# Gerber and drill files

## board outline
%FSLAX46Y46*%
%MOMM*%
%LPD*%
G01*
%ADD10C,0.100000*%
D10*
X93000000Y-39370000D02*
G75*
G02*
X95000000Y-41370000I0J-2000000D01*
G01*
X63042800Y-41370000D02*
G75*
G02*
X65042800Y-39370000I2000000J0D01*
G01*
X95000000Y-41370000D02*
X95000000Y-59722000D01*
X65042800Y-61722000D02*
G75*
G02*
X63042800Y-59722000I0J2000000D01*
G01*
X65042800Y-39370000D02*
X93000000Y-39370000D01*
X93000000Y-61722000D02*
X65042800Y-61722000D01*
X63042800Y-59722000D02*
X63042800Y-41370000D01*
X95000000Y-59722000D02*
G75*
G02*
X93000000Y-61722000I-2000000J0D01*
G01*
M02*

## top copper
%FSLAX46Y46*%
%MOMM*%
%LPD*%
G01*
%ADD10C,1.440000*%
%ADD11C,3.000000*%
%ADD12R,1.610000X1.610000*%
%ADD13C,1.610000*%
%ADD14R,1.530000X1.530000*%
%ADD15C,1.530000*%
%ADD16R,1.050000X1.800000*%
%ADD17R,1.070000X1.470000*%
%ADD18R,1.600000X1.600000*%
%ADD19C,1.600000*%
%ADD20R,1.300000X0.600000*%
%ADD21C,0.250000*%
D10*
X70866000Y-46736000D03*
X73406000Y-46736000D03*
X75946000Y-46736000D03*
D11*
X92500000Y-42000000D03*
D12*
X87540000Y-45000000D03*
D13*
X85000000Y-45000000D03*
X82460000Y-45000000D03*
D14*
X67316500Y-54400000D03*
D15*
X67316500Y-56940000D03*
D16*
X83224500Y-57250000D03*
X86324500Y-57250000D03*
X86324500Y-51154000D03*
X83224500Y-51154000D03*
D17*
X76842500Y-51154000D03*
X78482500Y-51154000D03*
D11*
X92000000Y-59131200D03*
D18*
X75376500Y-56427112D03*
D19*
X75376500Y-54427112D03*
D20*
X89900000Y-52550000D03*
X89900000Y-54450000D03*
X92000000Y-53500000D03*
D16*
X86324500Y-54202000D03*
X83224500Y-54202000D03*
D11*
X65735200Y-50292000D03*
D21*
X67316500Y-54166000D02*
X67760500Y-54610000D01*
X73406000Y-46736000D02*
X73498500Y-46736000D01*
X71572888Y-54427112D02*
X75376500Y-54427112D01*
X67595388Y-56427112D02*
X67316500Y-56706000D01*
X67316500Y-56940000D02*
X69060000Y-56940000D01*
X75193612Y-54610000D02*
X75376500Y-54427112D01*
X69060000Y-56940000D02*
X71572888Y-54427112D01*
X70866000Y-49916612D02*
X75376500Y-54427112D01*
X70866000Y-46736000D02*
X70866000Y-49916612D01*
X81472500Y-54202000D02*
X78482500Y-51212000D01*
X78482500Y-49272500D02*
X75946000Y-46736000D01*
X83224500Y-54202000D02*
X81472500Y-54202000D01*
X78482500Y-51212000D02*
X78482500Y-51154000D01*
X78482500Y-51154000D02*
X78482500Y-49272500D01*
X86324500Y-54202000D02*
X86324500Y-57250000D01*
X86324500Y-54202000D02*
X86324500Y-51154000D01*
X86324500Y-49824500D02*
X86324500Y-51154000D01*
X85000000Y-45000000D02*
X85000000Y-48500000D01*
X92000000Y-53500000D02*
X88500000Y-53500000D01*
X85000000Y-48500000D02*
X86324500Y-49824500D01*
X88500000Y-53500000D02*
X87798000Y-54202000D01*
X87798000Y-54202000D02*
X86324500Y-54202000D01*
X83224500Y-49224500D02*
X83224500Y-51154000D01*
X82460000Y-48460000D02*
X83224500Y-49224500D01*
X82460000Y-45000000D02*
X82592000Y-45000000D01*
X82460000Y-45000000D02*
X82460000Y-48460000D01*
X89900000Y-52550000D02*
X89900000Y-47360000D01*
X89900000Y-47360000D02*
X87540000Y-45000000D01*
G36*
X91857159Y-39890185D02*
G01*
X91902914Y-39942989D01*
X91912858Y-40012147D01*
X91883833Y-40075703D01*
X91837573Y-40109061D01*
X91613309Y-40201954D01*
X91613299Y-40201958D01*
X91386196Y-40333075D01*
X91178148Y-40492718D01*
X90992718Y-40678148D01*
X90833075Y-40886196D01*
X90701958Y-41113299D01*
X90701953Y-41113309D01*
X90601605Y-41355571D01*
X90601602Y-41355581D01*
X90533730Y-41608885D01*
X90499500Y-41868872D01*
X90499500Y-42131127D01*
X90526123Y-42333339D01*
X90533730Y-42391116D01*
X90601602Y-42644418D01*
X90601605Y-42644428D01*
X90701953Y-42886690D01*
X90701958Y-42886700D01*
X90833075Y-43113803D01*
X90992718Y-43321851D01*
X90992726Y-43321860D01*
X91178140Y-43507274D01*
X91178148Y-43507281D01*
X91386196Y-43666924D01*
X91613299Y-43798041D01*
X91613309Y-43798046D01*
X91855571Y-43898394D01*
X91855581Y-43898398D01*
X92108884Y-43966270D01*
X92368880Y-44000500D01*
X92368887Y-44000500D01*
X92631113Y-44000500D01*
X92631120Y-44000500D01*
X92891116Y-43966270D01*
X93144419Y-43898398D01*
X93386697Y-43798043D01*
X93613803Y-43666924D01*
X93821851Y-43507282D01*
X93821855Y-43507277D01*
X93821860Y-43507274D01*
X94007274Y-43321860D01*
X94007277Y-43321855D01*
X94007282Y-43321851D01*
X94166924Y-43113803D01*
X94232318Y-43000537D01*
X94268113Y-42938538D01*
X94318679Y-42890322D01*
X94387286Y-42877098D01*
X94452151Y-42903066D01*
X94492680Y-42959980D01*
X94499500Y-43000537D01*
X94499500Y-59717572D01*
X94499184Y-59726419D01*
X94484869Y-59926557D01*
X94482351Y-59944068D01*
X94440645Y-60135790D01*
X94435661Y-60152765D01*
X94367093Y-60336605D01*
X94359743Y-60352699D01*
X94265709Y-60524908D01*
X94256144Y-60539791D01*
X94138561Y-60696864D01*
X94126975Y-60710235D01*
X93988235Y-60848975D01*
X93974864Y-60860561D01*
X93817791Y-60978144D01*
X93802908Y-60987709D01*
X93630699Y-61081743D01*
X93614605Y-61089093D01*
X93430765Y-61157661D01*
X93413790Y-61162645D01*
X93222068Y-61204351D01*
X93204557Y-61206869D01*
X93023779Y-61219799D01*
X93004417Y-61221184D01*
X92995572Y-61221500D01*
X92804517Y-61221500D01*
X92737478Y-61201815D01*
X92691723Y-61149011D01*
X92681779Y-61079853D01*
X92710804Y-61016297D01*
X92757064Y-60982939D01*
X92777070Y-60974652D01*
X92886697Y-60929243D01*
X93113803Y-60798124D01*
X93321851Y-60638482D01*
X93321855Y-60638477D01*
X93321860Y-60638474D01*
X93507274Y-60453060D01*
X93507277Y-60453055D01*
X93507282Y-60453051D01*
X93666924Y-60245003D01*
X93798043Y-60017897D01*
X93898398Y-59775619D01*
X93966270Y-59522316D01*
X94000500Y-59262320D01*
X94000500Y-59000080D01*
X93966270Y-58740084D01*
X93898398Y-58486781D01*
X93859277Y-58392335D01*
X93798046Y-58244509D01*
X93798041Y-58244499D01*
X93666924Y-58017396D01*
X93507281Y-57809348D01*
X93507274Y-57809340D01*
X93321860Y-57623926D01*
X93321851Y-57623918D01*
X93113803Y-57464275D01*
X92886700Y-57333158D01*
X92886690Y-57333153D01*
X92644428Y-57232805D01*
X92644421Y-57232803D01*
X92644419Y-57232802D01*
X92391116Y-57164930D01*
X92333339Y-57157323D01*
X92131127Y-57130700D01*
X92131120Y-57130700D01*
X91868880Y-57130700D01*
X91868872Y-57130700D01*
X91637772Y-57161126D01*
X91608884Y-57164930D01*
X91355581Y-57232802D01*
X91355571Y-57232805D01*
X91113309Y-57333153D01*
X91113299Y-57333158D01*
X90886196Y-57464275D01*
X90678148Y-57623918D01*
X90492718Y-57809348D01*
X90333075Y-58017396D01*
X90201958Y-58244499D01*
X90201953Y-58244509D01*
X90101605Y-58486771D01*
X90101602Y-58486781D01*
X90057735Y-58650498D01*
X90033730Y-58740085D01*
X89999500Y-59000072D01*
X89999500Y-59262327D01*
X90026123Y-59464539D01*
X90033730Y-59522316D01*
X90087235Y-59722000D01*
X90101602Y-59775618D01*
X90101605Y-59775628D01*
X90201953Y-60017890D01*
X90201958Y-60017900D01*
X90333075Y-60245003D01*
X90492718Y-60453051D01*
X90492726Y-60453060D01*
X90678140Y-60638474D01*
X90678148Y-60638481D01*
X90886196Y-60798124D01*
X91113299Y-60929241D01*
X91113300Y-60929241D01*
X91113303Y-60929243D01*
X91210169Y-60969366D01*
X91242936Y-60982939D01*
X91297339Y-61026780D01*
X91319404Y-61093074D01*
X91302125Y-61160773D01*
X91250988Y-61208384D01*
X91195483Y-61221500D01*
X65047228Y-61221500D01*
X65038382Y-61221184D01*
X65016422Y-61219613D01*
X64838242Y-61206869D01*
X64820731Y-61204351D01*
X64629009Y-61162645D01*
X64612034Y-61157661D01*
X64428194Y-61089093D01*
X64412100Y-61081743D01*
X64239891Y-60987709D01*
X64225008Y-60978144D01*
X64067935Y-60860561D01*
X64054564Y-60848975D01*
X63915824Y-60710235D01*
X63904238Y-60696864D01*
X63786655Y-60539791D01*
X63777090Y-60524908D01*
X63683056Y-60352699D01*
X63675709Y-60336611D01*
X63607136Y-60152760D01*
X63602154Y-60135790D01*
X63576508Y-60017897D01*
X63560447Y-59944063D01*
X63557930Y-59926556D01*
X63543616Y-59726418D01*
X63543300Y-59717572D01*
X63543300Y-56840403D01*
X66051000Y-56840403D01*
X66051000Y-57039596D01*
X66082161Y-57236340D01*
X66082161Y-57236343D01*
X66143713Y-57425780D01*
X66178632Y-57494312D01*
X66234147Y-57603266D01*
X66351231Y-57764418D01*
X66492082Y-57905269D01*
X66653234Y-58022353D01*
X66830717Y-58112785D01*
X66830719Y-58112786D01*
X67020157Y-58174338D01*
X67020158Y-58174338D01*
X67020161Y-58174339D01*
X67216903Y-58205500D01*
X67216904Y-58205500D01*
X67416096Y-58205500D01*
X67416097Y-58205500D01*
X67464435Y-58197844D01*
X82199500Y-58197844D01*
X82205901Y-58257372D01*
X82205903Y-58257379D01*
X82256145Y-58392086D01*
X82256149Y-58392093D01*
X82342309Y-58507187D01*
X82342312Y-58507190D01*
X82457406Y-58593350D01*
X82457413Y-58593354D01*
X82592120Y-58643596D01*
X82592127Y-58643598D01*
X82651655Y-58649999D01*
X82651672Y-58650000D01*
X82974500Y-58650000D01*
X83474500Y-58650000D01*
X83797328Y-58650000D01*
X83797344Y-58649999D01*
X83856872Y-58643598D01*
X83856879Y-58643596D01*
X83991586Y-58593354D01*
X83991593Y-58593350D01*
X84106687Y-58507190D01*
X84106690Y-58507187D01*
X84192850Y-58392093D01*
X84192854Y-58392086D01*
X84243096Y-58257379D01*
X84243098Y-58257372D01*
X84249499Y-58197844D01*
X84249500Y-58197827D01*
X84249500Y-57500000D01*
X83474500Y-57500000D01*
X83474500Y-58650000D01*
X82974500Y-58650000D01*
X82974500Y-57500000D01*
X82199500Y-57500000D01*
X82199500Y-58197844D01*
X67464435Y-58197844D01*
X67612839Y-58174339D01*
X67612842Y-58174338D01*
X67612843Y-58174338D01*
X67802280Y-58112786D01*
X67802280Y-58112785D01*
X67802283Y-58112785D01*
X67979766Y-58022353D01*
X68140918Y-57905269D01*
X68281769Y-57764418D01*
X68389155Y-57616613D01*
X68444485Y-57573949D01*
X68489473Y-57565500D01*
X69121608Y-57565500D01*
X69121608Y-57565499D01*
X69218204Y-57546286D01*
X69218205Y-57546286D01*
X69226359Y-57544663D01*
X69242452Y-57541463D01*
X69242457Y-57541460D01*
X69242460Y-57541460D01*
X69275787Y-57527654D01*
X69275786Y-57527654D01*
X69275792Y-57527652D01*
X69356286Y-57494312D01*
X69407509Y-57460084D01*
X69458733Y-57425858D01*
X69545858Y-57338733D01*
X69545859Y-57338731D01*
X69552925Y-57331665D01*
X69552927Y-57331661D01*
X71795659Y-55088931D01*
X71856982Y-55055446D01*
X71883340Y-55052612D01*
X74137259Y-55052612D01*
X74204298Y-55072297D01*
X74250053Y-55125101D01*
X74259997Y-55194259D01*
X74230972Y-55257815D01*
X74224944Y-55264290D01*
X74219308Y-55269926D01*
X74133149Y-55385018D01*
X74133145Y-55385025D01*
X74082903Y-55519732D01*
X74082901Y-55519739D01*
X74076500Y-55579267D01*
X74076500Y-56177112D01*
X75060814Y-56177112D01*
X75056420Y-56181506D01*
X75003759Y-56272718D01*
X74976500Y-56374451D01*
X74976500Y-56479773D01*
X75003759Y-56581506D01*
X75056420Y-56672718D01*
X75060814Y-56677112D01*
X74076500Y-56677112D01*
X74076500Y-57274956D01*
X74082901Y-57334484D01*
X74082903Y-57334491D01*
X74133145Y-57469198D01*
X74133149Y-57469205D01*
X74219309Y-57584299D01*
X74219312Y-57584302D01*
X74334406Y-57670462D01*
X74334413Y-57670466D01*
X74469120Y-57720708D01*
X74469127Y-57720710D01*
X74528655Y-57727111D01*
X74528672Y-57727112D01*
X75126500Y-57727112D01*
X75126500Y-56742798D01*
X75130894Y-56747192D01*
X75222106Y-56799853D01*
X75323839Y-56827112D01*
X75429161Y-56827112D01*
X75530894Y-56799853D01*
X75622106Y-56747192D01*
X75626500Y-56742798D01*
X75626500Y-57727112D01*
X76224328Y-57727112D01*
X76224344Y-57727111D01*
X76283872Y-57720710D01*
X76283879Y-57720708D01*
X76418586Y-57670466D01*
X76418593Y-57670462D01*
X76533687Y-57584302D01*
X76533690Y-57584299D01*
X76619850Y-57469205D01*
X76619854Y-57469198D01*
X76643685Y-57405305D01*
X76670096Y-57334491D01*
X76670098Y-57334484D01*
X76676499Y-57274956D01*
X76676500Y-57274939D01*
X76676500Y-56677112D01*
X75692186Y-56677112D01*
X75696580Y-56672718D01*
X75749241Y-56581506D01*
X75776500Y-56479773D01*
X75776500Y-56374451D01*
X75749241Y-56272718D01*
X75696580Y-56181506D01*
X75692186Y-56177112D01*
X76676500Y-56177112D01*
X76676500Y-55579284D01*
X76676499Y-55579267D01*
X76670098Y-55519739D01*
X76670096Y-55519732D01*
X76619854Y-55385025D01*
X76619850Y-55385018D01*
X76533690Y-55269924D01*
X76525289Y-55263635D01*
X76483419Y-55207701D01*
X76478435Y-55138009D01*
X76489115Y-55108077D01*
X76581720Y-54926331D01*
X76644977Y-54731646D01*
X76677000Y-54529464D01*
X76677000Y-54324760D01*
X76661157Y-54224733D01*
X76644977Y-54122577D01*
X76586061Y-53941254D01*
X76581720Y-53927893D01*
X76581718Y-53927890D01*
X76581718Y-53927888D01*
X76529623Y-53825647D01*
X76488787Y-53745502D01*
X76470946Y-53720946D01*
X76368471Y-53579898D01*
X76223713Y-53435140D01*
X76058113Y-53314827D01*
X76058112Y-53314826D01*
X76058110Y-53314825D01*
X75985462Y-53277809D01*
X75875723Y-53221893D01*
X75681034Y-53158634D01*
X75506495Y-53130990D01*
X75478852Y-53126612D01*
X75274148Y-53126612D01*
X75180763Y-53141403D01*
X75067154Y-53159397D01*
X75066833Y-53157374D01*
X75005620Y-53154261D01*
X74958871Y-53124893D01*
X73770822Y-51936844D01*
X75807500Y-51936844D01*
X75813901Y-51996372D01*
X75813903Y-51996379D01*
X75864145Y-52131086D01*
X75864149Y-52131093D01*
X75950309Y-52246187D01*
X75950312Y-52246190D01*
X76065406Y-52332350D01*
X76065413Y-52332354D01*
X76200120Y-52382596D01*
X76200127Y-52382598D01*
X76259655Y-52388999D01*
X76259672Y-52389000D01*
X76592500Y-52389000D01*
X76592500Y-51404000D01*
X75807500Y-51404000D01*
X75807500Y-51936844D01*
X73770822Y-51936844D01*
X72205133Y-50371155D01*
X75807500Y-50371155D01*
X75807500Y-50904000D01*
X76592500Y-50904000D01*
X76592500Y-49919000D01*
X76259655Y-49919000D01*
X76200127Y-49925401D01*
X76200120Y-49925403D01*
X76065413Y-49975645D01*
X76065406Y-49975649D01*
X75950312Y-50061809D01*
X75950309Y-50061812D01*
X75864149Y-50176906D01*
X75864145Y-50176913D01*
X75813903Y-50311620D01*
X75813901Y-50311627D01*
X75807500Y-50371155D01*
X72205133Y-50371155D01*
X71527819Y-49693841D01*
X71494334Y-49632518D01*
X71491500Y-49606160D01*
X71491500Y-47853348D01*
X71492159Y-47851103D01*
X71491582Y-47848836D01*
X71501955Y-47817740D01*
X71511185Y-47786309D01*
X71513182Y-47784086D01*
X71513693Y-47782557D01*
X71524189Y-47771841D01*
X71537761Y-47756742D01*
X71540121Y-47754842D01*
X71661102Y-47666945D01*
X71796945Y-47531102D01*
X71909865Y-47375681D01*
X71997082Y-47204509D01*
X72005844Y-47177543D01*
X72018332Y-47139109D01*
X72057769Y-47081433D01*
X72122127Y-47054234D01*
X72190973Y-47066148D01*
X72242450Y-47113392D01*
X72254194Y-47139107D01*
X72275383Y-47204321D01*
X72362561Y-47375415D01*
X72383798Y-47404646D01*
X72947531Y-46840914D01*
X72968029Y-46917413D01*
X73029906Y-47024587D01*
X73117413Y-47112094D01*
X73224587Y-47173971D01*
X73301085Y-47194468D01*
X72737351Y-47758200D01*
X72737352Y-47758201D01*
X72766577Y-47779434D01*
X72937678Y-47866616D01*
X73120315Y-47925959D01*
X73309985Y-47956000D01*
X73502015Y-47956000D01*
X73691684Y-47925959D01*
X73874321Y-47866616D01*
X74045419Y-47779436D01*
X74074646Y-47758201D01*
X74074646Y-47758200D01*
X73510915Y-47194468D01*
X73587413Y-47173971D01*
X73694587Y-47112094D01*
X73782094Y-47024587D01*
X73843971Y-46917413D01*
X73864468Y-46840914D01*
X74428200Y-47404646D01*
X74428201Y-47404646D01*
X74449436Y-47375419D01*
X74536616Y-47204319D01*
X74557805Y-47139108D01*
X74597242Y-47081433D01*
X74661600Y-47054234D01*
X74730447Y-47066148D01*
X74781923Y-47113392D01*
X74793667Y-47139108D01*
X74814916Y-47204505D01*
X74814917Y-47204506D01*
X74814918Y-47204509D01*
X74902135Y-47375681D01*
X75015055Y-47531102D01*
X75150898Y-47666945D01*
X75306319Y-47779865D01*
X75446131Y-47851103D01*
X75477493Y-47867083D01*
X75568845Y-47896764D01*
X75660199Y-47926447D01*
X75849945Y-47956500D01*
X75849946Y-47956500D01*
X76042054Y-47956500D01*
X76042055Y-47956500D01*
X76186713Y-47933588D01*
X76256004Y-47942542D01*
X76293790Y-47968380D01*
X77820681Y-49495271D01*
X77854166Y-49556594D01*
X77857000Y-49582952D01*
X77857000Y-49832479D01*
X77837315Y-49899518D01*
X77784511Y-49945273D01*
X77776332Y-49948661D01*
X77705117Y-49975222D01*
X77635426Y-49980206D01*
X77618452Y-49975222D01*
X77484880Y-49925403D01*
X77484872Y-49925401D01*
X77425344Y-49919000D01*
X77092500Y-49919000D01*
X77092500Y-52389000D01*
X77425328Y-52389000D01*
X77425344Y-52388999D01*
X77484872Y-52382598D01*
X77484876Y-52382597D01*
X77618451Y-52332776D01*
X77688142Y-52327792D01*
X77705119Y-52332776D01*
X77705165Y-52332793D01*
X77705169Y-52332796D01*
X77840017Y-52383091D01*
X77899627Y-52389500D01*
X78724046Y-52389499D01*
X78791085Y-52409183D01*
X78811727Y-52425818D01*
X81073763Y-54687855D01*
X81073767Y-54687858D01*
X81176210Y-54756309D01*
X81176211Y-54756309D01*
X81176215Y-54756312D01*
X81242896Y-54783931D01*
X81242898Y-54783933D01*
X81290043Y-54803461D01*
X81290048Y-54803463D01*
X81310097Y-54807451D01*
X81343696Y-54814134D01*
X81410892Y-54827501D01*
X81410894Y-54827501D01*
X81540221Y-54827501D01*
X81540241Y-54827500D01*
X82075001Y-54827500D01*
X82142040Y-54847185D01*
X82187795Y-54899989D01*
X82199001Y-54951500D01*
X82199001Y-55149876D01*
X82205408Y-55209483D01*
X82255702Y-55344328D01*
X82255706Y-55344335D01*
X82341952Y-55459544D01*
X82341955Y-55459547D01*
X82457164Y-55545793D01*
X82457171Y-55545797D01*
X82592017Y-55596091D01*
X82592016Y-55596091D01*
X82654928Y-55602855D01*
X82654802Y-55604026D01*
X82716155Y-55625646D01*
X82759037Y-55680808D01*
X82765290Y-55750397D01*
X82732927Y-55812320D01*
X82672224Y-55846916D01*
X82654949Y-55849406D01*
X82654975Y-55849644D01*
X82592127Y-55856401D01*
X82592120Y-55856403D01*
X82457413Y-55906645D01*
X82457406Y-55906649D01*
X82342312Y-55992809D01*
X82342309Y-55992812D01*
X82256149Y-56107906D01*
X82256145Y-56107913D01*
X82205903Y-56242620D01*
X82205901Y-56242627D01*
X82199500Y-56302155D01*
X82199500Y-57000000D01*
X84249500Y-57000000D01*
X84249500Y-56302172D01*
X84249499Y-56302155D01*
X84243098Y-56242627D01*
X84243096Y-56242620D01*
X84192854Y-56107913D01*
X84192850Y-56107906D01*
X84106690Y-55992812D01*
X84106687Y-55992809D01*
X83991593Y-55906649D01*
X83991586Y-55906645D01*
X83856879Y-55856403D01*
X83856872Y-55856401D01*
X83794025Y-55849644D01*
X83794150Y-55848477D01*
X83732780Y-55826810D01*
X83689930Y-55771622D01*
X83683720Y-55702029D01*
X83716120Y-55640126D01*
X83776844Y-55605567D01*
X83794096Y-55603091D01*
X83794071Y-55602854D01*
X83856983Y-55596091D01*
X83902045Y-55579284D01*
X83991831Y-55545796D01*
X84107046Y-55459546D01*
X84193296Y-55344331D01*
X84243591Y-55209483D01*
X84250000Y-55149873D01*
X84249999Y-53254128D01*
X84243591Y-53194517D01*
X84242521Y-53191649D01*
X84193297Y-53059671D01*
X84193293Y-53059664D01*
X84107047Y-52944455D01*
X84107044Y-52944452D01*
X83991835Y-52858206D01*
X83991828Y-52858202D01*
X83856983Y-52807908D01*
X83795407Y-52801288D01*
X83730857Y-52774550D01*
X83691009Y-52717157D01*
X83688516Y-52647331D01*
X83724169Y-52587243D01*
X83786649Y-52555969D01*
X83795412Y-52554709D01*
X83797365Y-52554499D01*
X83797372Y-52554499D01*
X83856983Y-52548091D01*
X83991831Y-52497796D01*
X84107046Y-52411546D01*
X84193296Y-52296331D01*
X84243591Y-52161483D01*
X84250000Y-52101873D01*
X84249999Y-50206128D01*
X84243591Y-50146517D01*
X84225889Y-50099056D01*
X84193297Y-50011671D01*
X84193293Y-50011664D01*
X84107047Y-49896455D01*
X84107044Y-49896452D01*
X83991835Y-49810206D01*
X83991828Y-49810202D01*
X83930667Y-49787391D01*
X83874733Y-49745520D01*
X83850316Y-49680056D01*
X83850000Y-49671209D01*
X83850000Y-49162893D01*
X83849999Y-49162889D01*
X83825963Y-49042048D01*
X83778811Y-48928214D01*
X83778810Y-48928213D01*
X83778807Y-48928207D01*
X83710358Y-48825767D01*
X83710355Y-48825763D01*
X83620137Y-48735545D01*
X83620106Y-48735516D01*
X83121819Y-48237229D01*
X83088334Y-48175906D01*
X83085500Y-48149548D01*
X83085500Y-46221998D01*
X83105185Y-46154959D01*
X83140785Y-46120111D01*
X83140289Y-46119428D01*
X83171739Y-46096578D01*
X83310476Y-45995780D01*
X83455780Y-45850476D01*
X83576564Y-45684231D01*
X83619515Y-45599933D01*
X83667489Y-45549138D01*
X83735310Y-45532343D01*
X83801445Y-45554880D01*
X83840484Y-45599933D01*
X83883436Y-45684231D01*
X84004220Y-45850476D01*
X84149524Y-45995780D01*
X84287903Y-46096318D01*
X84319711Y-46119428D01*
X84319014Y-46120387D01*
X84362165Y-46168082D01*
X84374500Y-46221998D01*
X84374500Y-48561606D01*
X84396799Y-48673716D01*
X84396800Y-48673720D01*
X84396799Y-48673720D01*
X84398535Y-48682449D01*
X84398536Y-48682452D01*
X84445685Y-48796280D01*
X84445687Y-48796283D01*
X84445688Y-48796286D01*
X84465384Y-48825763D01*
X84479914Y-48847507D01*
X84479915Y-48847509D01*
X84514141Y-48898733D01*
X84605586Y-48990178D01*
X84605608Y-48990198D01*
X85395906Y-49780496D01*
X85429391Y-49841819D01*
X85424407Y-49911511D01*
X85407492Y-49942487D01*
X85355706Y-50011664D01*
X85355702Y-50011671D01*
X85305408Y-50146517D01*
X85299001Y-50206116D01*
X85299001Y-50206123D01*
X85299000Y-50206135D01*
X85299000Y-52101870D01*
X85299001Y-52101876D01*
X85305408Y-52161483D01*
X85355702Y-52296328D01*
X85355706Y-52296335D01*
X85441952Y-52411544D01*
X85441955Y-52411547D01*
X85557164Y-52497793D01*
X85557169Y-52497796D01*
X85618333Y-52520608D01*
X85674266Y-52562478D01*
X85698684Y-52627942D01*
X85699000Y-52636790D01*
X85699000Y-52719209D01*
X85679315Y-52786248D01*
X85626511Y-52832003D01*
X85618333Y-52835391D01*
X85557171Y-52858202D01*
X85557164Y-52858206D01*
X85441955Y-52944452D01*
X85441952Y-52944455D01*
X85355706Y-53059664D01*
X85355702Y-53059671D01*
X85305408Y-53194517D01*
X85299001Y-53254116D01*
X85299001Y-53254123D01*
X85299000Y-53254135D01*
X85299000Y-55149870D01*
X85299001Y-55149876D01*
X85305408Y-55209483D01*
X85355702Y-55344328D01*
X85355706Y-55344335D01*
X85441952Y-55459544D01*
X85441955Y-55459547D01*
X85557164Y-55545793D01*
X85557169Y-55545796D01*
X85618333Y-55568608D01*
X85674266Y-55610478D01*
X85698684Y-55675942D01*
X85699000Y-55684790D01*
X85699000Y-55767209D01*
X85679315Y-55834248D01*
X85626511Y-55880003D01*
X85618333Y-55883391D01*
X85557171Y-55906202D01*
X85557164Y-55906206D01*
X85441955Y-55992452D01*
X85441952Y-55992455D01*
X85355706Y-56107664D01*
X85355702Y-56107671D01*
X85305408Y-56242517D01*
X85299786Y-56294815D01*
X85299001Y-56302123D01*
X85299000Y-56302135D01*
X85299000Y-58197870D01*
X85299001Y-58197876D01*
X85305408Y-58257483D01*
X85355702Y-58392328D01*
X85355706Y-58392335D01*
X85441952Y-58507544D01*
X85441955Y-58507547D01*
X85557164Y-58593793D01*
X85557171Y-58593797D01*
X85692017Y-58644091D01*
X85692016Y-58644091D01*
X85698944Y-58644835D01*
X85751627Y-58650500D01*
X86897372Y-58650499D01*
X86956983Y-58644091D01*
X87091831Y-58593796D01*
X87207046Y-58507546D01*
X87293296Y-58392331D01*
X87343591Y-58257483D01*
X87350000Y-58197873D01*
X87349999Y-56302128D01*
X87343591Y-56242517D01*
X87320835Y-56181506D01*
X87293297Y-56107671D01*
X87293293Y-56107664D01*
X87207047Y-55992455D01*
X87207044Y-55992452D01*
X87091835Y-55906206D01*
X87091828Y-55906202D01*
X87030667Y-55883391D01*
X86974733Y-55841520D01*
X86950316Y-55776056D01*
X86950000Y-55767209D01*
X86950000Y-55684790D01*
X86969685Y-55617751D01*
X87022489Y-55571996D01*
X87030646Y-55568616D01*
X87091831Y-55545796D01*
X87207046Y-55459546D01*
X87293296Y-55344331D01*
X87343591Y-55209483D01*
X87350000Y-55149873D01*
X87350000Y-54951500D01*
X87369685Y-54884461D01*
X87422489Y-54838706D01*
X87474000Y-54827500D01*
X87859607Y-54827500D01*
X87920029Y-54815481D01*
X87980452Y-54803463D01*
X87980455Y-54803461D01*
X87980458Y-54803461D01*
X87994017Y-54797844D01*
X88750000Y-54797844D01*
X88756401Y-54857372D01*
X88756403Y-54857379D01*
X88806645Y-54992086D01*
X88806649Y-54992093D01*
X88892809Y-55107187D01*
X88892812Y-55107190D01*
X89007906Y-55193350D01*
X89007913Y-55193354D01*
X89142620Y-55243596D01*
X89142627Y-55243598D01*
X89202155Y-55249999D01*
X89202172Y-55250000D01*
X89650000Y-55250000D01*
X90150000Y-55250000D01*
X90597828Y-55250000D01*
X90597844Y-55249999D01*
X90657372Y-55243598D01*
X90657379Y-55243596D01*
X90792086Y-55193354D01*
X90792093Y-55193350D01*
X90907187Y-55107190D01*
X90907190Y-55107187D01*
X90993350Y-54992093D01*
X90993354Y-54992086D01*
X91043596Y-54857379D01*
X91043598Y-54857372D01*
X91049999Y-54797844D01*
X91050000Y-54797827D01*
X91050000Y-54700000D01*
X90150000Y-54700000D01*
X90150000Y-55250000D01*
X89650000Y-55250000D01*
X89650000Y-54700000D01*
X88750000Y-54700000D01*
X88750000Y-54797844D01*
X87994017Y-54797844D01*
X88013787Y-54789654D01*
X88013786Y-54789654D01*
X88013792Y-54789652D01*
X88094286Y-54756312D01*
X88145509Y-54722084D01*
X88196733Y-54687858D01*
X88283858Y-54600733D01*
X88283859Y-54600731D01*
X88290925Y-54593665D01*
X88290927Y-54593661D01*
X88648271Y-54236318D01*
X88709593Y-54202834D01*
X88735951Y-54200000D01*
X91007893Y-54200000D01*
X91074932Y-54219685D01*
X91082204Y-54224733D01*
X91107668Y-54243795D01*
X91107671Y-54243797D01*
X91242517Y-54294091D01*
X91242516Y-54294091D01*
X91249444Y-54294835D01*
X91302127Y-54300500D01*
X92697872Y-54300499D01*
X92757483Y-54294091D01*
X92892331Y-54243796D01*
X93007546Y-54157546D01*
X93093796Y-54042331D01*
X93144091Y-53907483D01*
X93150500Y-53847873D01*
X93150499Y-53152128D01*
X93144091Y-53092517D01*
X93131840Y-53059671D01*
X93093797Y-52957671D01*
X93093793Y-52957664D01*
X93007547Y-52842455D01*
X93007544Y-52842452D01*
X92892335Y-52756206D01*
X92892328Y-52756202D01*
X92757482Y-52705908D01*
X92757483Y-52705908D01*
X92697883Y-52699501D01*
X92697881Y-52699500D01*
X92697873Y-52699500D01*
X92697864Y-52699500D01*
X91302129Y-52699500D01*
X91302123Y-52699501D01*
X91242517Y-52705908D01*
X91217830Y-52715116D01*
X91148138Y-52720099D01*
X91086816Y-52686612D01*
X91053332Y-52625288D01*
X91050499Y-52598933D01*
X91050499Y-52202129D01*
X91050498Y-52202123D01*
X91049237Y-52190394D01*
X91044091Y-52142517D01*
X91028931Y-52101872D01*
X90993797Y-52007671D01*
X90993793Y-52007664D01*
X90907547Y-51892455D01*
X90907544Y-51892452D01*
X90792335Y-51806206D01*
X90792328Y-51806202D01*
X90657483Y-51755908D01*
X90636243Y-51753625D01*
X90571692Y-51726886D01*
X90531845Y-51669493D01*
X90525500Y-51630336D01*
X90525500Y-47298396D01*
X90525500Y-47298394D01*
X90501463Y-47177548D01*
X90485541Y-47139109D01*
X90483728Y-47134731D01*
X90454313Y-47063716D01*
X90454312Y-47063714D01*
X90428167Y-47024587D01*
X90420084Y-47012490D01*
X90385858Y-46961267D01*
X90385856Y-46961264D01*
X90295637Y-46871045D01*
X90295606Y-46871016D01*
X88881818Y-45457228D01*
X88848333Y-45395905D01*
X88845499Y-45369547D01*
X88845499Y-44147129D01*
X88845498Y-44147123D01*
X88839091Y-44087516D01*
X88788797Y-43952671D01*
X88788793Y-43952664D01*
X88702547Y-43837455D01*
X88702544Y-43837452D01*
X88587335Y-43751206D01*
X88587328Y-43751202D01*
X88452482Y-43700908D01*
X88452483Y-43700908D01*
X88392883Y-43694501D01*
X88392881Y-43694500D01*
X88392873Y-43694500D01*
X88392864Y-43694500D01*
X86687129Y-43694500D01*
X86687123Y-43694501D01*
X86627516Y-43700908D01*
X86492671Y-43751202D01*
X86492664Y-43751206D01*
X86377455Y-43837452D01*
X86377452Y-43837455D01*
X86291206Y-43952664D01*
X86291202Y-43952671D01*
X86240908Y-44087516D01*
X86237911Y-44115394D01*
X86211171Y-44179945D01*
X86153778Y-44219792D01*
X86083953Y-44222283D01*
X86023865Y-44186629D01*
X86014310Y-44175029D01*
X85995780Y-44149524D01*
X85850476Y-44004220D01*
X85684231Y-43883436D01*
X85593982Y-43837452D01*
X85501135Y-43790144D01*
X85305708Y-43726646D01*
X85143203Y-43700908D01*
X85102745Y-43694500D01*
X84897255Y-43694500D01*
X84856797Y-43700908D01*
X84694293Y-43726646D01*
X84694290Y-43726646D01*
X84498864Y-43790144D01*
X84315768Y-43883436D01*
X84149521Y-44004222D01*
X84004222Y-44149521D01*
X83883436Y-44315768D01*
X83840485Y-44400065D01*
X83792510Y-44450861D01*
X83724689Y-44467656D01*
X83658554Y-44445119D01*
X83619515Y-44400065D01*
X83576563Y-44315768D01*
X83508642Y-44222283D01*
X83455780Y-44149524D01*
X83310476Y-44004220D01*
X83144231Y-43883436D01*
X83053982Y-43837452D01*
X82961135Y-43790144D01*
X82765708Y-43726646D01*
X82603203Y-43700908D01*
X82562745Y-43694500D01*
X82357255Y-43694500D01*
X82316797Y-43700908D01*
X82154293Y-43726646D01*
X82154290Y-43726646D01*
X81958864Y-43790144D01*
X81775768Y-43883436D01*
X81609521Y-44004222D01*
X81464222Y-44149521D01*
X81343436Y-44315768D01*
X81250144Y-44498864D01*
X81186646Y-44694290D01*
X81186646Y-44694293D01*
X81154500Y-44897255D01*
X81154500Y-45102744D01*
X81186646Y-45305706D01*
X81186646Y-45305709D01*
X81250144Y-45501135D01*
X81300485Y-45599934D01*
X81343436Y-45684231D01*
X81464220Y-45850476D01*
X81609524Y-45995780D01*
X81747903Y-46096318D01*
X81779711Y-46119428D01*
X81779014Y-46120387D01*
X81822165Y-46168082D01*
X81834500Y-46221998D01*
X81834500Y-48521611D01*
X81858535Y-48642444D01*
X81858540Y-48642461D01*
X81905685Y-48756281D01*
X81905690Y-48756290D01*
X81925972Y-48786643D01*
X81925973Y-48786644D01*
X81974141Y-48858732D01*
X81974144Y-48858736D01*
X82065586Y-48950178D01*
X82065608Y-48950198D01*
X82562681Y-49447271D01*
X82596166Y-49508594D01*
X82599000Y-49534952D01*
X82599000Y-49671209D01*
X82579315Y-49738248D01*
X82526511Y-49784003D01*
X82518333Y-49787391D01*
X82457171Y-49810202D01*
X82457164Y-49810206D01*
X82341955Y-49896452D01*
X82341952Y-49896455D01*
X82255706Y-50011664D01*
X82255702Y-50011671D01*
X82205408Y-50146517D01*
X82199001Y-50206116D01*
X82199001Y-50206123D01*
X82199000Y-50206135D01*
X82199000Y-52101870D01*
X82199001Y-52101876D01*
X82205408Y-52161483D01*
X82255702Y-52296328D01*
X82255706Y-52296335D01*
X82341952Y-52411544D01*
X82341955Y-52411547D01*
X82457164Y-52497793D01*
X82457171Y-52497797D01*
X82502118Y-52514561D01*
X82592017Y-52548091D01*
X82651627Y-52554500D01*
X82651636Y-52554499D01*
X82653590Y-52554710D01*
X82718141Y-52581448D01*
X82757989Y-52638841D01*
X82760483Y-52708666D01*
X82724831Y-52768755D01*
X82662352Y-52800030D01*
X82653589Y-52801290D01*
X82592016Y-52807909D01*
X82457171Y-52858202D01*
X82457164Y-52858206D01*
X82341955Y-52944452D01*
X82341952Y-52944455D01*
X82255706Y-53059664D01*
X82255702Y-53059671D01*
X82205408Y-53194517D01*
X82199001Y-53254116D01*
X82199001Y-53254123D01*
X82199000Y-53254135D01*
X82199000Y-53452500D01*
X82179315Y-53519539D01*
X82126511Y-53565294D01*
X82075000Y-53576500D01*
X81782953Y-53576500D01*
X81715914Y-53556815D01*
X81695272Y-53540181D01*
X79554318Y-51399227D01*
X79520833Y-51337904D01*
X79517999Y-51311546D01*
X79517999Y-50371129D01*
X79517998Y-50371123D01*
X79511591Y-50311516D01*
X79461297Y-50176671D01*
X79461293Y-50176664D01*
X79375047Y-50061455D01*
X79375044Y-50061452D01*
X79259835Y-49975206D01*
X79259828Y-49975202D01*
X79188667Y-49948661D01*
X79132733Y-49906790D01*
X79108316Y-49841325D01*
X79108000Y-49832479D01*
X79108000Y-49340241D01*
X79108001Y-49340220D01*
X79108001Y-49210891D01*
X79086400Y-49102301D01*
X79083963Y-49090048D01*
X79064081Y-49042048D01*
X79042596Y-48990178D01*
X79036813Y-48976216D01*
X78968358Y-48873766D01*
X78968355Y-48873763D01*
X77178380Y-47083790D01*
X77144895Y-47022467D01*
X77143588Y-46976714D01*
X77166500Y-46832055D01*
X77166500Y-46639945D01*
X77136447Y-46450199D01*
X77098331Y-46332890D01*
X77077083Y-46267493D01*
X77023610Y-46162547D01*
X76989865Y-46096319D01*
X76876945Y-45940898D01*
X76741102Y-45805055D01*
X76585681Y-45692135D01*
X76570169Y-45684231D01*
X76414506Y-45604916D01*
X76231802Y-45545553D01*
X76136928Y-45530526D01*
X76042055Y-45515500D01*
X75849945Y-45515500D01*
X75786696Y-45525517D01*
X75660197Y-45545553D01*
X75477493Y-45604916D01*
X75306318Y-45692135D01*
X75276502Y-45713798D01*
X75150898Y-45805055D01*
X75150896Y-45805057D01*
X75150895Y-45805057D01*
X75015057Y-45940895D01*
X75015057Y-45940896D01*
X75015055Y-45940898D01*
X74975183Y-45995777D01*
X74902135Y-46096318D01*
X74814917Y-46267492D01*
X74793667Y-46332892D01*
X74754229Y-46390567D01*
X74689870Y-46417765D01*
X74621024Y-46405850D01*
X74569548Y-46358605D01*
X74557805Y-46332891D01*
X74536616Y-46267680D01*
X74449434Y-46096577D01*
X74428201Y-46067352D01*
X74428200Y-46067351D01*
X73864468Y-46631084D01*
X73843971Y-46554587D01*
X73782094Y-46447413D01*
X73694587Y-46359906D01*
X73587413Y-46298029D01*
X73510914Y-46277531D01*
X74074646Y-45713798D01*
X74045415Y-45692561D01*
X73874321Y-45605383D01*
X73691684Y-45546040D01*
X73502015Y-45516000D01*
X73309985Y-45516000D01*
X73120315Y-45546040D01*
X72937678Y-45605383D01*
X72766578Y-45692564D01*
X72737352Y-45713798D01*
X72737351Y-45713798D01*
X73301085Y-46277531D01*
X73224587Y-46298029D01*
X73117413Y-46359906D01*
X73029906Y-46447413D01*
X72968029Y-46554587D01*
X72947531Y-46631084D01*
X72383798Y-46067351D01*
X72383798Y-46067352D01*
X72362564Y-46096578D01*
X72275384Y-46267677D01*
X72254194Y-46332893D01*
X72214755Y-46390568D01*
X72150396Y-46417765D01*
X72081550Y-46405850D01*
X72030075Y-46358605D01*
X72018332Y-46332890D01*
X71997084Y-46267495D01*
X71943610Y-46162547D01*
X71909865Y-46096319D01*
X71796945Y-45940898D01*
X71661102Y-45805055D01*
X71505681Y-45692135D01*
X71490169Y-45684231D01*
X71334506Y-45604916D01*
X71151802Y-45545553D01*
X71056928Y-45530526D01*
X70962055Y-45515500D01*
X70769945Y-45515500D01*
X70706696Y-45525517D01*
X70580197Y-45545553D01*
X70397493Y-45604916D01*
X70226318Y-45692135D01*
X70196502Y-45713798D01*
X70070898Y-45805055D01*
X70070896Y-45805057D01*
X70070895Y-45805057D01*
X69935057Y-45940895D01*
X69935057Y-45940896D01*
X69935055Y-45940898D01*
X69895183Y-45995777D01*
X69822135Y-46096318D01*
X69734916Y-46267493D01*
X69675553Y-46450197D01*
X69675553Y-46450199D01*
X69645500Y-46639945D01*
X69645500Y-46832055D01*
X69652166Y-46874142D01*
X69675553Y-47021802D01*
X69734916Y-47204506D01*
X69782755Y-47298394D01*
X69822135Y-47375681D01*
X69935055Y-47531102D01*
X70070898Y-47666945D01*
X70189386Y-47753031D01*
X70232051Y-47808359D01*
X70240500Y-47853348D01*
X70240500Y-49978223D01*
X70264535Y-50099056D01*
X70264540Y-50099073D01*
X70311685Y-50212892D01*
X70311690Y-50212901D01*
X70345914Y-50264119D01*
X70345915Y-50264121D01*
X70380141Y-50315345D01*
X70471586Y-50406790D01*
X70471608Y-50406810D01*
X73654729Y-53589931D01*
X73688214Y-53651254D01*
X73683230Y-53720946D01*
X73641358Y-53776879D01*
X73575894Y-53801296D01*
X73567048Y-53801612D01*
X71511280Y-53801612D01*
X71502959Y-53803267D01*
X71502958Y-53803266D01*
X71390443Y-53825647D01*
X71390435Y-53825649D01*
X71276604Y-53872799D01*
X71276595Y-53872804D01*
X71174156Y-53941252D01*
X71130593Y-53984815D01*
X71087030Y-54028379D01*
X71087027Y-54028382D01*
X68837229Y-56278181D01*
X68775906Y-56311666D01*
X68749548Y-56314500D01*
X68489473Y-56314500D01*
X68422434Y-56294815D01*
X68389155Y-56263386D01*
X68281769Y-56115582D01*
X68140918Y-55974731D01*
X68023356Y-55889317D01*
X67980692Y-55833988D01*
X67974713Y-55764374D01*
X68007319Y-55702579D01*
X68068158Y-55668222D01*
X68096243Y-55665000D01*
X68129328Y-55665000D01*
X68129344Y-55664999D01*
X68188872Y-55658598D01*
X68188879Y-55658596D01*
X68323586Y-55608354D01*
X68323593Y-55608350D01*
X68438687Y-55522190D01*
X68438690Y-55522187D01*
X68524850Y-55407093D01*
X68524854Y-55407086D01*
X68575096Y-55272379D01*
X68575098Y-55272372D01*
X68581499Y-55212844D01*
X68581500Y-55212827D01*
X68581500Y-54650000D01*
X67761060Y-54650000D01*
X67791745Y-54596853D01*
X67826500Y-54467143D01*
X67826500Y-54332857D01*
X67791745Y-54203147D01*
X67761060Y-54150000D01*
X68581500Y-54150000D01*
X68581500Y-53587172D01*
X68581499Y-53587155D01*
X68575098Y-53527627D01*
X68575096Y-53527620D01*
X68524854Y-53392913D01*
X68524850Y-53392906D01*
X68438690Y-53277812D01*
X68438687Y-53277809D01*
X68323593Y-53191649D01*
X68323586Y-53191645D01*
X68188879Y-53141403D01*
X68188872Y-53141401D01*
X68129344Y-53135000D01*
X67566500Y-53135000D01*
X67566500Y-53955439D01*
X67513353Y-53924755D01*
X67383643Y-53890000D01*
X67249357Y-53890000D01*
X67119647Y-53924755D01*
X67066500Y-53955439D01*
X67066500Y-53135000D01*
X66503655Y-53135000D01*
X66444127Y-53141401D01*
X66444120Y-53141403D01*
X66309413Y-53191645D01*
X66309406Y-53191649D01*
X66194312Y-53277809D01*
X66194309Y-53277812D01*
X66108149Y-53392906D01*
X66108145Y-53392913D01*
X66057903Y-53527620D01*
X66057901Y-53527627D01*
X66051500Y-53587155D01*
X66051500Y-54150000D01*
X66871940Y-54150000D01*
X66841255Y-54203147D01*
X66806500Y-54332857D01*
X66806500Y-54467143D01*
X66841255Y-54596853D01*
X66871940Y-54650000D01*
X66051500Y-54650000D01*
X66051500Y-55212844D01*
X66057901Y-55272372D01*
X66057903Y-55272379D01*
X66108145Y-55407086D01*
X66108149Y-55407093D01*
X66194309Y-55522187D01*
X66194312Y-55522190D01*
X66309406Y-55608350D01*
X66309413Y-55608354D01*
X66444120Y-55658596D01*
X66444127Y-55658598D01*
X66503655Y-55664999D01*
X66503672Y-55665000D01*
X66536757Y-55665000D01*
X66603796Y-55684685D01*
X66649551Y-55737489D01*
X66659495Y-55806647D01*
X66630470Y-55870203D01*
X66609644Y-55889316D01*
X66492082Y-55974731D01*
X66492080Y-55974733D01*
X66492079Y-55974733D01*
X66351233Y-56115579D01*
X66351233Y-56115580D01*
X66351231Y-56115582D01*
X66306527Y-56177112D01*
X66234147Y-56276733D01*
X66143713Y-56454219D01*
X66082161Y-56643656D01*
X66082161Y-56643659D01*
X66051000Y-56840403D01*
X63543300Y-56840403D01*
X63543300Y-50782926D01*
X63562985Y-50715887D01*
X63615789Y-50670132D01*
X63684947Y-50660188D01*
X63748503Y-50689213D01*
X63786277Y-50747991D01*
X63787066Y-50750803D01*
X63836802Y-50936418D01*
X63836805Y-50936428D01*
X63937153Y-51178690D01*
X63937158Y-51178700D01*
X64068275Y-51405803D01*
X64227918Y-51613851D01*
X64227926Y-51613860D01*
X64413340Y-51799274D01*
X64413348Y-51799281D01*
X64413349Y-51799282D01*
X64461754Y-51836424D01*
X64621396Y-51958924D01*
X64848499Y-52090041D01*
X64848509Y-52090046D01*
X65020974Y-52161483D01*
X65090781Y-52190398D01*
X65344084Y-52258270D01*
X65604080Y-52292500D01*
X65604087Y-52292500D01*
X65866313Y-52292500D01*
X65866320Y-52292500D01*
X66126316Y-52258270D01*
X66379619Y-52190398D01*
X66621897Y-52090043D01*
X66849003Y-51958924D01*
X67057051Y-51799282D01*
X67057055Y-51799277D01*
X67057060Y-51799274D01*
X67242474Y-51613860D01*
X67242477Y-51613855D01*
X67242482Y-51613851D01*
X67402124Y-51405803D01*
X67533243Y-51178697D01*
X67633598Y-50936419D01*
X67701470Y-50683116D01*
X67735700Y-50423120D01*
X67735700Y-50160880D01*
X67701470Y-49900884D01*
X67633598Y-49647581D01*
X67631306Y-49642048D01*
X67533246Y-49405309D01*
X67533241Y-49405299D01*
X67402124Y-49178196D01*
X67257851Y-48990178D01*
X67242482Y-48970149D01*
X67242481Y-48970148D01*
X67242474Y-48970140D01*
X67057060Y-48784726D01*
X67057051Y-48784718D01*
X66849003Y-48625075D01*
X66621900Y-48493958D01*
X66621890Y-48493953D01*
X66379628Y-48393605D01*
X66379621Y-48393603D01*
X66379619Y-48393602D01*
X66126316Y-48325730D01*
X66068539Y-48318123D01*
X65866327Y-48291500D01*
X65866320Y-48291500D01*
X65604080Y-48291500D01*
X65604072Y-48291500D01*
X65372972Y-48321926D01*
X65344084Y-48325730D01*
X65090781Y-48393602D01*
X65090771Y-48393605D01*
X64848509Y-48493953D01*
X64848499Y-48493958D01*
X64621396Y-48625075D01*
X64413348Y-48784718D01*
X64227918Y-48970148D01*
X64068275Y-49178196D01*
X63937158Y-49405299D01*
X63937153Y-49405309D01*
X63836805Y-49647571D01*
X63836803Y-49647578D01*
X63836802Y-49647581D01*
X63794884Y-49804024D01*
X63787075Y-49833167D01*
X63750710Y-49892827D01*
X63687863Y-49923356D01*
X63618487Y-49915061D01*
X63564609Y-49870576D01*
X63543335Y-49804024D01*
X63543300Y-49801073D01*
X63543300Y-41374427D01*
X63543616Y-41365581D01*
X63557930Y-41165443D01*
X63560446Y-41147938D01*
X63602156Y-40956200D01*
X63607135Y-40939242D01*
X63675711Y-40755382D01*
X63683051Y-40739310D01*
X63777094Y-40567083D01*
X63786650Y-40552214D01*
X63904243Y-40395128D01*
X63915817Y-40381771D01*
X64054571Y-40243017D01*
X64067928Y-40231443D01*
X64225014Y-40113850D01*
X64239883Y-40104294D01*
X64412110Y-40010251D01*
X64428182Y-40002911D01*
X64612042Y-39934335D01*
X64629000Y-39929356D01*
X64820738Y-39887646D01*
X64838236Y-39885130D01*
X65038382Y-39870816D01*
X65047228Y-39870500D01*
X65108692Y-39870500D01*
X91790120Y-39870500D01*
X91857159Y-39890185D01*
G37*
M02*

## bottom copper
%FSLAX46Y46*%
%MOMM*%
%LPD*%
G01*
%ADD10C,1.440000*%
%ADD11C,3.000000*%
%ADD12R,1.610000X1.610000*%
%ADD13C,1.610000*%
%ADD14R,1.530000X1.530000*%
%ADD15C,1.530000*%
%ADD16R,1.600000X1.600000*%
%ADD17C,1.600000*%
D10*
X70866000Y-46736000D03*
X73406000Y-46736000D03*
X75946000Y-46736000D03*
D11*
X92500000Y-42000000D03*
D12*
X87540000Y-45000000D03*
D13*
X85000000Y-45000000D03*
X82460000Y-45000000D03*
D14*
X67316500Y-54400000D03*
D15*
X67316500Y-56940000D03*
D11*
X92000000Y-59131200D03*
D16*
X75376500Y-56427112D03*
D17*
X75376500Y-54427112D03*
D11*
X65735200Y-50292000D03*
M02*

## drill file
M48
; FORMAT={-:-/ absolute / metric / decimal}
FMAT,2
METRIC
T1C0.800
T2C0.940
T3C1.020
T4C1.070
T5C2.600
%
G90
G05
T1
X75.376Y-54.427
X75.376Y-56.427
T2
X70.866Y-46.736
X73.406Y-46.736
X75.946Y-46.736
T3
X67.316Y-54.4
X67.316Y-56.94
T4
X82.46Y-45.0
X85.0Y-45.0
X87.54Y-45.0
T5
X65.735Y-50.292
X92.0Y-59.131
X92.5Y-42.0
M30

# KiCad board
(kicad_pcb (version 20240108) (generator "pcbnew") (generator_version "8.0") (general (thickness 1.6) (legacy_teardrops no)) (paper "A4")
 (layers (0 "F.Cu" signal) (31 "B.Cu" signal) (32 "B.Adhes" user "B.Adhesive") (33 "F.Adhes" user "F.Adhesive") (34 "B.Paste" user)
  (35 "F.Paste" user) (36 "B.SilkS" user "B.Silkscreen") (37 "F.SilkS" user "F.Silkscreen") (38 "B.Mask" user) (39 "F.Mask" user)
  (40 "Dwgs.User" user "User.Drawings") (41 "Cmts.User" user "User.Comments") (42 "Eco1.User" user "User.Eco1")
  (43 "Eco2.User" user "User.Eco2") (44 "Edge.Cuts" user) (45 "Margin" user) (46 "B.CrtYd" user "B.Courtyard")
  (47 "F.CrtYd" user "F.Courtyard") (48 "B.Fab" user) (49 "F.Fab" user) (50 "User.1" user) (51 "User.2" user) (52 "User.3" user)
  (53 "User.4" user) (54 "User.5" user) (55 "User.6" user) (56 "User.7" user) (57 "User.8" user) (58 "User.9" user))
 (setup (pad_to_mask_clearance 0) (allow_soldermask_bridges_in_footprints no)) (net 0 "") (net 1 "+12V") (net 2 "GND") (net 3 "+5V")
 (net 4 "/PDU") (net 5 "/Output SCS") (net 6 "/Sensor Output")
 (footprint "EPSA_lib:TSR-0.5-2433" (layer "F.Cu") (at 67.656 48.736)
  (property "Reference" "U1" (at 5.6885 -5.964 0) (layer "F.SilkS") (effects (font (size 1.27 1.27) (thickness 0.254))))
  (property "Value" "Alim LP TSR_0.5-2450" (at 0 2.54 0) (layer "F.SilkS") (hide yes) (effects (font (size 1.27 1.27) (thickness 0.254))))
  (pad "1" thru_hole circle (at 3.21 -2) (size 1.44 1.44) (drill 0.94) (layers "*.Cu" "*.Mask") (remove_unused_layers no) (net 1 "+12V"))
  (pad "2" thru_hole circle (at 5.75 -2) (size 1.44 1.44) (drill 0.94) (layers "*.Cu" "*.Mask") (remove_unused_layers no) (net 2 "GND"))
  (pad "3" thru_hole circle (at 8.29 -2) (size 1.44 1.44) (drill 0.94) (layers "*.Cu" "*.Mask") (remove_unused_layers no) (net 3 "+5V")))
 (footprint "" (layer "F.Cu") (at 92.5 42)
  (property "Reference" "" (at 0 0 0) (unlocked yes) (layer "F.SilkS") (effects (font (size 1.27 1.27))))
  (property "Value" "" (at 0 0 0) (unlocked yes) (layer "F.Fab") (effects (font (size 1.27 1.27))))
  (pad "1" thru_hole circle (at 0 0) (size 3 3) (drill 2.6) (layers "*.Cu" "*.Mask") (remove_unused_layers no)))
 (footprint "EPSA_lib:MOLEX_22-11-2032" (layer "F.Cu") (at 87.54 45 180)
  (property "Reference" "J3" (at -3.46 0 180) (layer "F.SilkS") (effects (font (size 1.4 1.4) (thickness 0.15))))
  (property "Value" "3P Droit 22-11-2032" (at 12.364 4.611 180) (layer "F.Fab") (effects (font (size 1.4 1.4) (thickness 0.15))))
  (pad "1" thru_hole rect (at 0 0 180) (size 1.61 1.61) (drill 1.07) (layers "*.Cu" "*.Mask") (remove_unused_layers no) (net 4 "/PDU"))
  (pad "2" thru_hole circle (at 2.54 0 180) (size 1.61 1.61) (drill 1.07) (layers "*.Cu" "*.Mask") (remove_unused_layers no)
   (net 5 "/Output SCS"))
  (pad "3" thru_hole circle (at 5.08 0 180) (size 1.61 1.61) (drill 1.07) (layers "*.Cu" "*.Mask") (remove_unused_layers no)
   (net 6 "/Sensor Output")))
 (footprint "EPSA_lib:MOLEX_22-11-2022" (layer "F.Cu") (at 67.3165 54.4 -90)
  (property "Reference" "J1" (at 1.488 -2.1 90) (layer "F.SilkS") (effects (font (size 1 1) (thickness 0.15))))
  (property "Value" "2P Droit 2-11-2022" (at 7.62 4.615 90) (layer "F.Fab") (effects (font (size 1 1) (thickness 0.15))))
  (pad "1" thru_hole rect (at 0 0 270) (size 1.53 1.53) (drill 1.02) (layers "*.Cu" "*.Mask") (remove_unused_layers no) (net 2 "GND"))
  (pad "2" thru_hole circle (at 2.54 0 270) (size 1.53 1.53) (drill 1.02) (layers "*.Cu" "*.Mask") (remove_unused_layers no) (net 1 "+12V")))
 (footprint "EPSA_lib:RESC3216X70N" (layer "F.Cu") (at 84.7745 57.25)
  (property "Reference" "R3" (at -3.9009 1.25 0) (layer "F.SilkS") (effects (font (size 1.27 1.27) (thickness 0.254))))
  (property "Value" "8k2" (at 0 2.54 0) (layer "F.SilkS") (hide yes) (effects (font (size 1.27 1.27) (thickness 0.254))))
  (pad "1" smd rect (at -1.55 0) (size 1.05 1.8) (layers "F.Cu" "F.Paste" "F.Mask") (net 2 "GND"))
  (pad "2" smd rect (at 1.55 0) (size 1.05 1.8) (layers "F.Cu" "F.Paste" "F.Mask") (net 5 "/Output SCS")))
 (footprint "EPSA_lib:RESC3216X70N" (layer "F.Cu") (at 84.7745 51.154 180)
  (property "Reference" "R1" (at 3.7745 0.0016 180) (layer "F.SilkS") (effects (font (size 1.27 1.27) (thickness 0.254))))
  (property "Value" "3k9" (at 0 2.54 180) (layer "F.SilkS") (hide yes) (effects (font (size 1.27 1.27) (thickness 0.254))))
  (pad "1" smd rect (at -1.55 0 180) (size 1.05 1.8) (layers "F.Cu" "F.Paste" "F.Mask") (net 5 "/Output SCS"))
  (pad "2" smd rect (at 1.55 0 180) (size 1.05 1.8) (layers "F.Cu" "F.Paste" "F.Mask") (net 6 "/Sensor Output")))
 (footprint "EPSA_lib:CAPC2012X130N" (layer "F.Cu") (at 77.6625 51.154)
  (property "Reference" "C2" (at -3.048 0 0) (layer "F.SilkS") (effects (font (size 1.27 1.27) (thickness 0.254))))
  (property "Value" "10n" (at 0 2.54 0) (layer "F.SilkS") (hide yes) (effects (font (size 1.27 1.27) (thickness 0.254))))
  (pad "1" smd rect (at -0.82 0) (size 1.07 1.47) (layers "F.Cu" "F.Paste" "F.Mask") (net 2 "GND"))
  (pad "2" smd rect (at 0.82 0) (size 1.07 1.47) (layers "F.Cu" "F.Paste" "F.Mask") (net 3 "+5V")))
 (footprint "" (layer "F.Cu") (at 92 59.1312)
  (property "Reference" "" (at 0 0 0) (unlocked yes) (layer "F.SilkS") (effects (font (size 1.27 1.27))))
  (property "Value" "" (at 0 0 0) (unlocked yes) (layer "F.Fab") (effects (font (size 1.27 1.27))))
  (pad "1" thru_hole circle (at 0 0) (size 3 3) (drill 2.6) (layers "*.Cu" "*.Mask") (remove_unused_layers no)))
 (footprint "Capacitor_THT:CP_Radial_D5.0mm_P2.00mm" (layer "F.Cu") (at 75.3765 56.427112 90)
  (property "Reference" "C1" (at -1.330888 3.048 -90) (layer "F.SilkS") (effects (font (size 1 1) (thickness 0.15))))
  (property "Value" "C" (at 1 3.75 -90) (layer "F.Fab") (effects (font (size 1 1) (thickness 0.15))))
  (pad "1" thru_hole rect (at 0 0 90) (size 1.6 1.6) (drill 0.8) (layers "*.Cu" "*.Mask") (remove_unused_layers no) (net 2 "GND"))
  (pad "2" thru_hole circle (at 2 0 90) (size 1.6 1.6) (drill 0.8) (layers "*.Cu" "*.Mask") (remove_unused_layers no) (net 1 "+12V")))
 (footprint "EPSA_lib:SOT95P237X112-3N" (layer "F.Cu") (at 90.95 53.5)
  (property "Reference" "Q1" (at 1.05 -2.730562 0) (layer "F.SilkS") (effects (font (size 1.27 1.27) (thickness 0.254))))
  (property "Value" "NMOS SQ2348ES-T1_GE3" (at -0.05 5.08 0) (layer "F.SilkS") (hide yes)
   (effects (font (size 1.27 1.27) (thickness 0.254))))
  (pad "1" smd rect (at -1.05 -0.95 90) (size 0.6 1.3) (layers "F.Cu" "F.Paste" "F.Mask") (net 4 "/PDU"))
  (pad "2" smd rect (at -1.05 0.95 90) (size 0.6 1.3) (layers "F.Cu" "F.Paste" "F.Mask") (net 2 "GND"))
  (pad "3" smd rect (at 1.05 0 90) (size 0.6 1.3) (layers "F.Cu" "F.Paste" "F.Mask") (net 5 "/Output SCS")))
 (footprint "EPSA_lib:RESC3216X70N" (layer "F.Cu") (at 84.7745 54.202 180)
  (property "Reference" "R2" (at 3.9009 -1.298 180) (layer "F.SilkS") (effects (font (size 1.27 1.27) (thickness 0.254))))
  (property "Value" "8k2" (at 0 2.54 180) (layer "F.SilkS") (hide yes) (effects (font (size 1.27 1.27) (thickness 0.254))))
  (pad "1" smd rect (at -1.55 0 180) (size 1.05 1.8) (layers "F.Cu" "F.Paste" "F.Mask") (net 5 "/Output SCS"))
  (pad "2" smd rect (at 1.55 0 180) (size 1.05 1.8) (layers "F.Cu" "F.Paste" "F.Mask") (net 3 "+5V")))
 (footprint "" (layer "F.Cu") (at 65.7352 50.292)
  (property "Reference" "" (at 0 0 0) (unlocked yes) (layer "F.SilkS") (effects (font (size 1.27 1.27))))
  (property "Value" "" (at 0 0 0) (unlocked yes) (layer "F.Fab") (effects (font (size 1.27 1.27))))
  (pad "1" thru_hole circle (at 0 0) (size 3 3) (drill 2.6) (layers "*.Cu" "*.Mask") (remove_unused_layers no)))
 (gr_arc (start 93 39.37) (mid 94.414214 39.955786) (end 95 41.37) (stroke (width 0.1) (type default)) (layer "Edge.Cuts"))
 (gr_arc (start 63.0428 41.37) (mid 63.628586 39.955786) (end 65.0428 39.37) (stroke (width 0.1) (type default)) (layer "Edge.Cuts"))
 (gr_line (start 95 41.37) (end 95 59.722) (stroke (width 0.1) (type default)) (layer "Edge.Cuts"))
 (gr_arc (start 65.0428 61.722) (mid 63.628586 61.136214) (end 63.0428 59.722) (stroke (width 0.1) (type default)) (layer "Edge.Cuts"))
 (gr_line (start 65.0428 39.37) (end 93 39.37) (stroke (width 0.1) (type default)) (layer "Edge.Cuts"))
 (gr_line (start 93 61.722) (end 65.0428 61.722) (stroke (width 0.1) (type default)) (layer "Edge.Cuts"))
 (gr_line (start 63.0428 59.722) (end 63.0428 41.37) (stroke (width 0.1) (type default)) (layer "Edge.Cuts"))
 (gr_arc (start 95 59.722) (mid 94.414214 61.136214) (end 93 61.722) (stroke (width 0.1) (type default)) (layer "Edge.Cuts"))
 (segment (start 67.3165 54.166) (end 67.7605 54.61) (width 0.25) (layer "F.Cu") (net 2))
 (segment (start 73.406 46.736) (end 73.4985 46.736) (width 0.25) (layer "F.Cu") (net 2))
 (segment (start 71.572888 54.427112) (end 75.3765 54.427112) (width 0.25) (layer "F.Cu") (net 1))
 (segment (start 67.595388 56.427112) (end 67.3165 56.706) (width 0.25) (layer "F.Cu") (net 1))
 (segment (start 67.3165 56.94) (end 69.06 56.94) (width 0.25) (layer "F.Cu") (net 1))
 (segment (start 75.193612 54.61) (end 75.3765 54.427112) (width 0.25) (layer "F.Cu") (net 1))
 (segment (start 69.06 56.94) (end 71.572888 54.427112) (width 0.25) (layer "F.Cu") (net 1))
 (segment (start 70.866 49.916612) (end 75.3765 54.427112) (width 0.25) (layer "F.Cu") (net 1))
 (segment (start 70.866 46.736) (end 70.866 49.916612) (width 0.25) (layer "F.Cu") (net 1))
 (segment (start 81.4725 54.202) (end 78.4825 51.212) (width 0.25) (layer "F.Cu") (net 3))
 (segment (start 78.4825 49.2725) (end 75.946 46.736) (width 0.25) (layer "F.Cu") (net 3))
 (segment (start 83.2245 54.202) (end 81.4725 54.202) (width 0.25) (layer "F.Cu") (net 3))
 (segment (start 78.4825 51.212) (end 78.4825 51.154) (width 0.25) (layer "F.Cu") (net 3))
 (segment (start 78.4825 51.154) (end 78.4825 49.2725) (width 0.25) (layer "F.Cu") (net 3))
 (segment (start 86.3245 54.202) (end 86.3245 57.25) (width 0.25) (layer "F.Cu") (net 5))
 (segment (start 86.3245 54.202) (end 86.3245 51.154) (width 0.25) (layer "F.Cu") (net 5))
 (segment (start 86.3245 49.8245) (end 86.3245 51.154) (width 0.25) (layer "F.Cu") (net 5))
 (segment (start 85 45) (end 85 48.5) (width 0.25) (layer "F.Cu") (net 5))
 (segment (start 92 53.5) (end 88.5 53.5) (width 0.25) (layer "F.Cu") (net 5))
 (segment (start 85 48.5) (end 86.3245 49.8245) (width 0.25) (layer "F.Cu") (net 5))
 (segment (start 88.5 53.5) (end 87.798 54.202) (width 0.25) (layer "F.Cu") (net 5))
 (segment (start 87.798 54.202) (end 86.3245 54.202) (width 0.25) (layer "F.Cu") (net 5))
 (segment (start 83.2245 49.2245) (end 83.2245 51.154) (width 0.25) (layer "F.Cu") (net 6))
 (segment (start 82.46 48.46) (end 83.2245 49.2245) (width 0.25) (layer "F.Cu") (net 6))
 (segment (start 82.46 45) (end 82.592 45) (width 0.25) (layer "F.Cu") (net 6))
 (segment (start 82.46 45) (end 82.46 48.46) (width 0.25) (layer "F.Cu") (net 6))
 (segment (start 89.9 52.55) (end 89.9 47.36) (width 0.25) (layer "F.Cu") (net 4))
 (segment (start 89.9 47.36) (end 87.54 45) (width 0.25) (layer "F.Cu") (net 4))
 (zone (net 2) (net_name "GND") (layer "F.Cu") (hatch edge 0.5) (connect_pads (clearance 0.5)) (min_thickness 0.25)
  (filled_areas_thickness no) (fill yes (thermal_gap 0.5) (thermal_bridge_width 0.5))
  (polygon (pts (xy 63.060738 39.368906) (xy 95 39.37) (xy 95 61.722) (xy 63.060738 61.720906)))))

